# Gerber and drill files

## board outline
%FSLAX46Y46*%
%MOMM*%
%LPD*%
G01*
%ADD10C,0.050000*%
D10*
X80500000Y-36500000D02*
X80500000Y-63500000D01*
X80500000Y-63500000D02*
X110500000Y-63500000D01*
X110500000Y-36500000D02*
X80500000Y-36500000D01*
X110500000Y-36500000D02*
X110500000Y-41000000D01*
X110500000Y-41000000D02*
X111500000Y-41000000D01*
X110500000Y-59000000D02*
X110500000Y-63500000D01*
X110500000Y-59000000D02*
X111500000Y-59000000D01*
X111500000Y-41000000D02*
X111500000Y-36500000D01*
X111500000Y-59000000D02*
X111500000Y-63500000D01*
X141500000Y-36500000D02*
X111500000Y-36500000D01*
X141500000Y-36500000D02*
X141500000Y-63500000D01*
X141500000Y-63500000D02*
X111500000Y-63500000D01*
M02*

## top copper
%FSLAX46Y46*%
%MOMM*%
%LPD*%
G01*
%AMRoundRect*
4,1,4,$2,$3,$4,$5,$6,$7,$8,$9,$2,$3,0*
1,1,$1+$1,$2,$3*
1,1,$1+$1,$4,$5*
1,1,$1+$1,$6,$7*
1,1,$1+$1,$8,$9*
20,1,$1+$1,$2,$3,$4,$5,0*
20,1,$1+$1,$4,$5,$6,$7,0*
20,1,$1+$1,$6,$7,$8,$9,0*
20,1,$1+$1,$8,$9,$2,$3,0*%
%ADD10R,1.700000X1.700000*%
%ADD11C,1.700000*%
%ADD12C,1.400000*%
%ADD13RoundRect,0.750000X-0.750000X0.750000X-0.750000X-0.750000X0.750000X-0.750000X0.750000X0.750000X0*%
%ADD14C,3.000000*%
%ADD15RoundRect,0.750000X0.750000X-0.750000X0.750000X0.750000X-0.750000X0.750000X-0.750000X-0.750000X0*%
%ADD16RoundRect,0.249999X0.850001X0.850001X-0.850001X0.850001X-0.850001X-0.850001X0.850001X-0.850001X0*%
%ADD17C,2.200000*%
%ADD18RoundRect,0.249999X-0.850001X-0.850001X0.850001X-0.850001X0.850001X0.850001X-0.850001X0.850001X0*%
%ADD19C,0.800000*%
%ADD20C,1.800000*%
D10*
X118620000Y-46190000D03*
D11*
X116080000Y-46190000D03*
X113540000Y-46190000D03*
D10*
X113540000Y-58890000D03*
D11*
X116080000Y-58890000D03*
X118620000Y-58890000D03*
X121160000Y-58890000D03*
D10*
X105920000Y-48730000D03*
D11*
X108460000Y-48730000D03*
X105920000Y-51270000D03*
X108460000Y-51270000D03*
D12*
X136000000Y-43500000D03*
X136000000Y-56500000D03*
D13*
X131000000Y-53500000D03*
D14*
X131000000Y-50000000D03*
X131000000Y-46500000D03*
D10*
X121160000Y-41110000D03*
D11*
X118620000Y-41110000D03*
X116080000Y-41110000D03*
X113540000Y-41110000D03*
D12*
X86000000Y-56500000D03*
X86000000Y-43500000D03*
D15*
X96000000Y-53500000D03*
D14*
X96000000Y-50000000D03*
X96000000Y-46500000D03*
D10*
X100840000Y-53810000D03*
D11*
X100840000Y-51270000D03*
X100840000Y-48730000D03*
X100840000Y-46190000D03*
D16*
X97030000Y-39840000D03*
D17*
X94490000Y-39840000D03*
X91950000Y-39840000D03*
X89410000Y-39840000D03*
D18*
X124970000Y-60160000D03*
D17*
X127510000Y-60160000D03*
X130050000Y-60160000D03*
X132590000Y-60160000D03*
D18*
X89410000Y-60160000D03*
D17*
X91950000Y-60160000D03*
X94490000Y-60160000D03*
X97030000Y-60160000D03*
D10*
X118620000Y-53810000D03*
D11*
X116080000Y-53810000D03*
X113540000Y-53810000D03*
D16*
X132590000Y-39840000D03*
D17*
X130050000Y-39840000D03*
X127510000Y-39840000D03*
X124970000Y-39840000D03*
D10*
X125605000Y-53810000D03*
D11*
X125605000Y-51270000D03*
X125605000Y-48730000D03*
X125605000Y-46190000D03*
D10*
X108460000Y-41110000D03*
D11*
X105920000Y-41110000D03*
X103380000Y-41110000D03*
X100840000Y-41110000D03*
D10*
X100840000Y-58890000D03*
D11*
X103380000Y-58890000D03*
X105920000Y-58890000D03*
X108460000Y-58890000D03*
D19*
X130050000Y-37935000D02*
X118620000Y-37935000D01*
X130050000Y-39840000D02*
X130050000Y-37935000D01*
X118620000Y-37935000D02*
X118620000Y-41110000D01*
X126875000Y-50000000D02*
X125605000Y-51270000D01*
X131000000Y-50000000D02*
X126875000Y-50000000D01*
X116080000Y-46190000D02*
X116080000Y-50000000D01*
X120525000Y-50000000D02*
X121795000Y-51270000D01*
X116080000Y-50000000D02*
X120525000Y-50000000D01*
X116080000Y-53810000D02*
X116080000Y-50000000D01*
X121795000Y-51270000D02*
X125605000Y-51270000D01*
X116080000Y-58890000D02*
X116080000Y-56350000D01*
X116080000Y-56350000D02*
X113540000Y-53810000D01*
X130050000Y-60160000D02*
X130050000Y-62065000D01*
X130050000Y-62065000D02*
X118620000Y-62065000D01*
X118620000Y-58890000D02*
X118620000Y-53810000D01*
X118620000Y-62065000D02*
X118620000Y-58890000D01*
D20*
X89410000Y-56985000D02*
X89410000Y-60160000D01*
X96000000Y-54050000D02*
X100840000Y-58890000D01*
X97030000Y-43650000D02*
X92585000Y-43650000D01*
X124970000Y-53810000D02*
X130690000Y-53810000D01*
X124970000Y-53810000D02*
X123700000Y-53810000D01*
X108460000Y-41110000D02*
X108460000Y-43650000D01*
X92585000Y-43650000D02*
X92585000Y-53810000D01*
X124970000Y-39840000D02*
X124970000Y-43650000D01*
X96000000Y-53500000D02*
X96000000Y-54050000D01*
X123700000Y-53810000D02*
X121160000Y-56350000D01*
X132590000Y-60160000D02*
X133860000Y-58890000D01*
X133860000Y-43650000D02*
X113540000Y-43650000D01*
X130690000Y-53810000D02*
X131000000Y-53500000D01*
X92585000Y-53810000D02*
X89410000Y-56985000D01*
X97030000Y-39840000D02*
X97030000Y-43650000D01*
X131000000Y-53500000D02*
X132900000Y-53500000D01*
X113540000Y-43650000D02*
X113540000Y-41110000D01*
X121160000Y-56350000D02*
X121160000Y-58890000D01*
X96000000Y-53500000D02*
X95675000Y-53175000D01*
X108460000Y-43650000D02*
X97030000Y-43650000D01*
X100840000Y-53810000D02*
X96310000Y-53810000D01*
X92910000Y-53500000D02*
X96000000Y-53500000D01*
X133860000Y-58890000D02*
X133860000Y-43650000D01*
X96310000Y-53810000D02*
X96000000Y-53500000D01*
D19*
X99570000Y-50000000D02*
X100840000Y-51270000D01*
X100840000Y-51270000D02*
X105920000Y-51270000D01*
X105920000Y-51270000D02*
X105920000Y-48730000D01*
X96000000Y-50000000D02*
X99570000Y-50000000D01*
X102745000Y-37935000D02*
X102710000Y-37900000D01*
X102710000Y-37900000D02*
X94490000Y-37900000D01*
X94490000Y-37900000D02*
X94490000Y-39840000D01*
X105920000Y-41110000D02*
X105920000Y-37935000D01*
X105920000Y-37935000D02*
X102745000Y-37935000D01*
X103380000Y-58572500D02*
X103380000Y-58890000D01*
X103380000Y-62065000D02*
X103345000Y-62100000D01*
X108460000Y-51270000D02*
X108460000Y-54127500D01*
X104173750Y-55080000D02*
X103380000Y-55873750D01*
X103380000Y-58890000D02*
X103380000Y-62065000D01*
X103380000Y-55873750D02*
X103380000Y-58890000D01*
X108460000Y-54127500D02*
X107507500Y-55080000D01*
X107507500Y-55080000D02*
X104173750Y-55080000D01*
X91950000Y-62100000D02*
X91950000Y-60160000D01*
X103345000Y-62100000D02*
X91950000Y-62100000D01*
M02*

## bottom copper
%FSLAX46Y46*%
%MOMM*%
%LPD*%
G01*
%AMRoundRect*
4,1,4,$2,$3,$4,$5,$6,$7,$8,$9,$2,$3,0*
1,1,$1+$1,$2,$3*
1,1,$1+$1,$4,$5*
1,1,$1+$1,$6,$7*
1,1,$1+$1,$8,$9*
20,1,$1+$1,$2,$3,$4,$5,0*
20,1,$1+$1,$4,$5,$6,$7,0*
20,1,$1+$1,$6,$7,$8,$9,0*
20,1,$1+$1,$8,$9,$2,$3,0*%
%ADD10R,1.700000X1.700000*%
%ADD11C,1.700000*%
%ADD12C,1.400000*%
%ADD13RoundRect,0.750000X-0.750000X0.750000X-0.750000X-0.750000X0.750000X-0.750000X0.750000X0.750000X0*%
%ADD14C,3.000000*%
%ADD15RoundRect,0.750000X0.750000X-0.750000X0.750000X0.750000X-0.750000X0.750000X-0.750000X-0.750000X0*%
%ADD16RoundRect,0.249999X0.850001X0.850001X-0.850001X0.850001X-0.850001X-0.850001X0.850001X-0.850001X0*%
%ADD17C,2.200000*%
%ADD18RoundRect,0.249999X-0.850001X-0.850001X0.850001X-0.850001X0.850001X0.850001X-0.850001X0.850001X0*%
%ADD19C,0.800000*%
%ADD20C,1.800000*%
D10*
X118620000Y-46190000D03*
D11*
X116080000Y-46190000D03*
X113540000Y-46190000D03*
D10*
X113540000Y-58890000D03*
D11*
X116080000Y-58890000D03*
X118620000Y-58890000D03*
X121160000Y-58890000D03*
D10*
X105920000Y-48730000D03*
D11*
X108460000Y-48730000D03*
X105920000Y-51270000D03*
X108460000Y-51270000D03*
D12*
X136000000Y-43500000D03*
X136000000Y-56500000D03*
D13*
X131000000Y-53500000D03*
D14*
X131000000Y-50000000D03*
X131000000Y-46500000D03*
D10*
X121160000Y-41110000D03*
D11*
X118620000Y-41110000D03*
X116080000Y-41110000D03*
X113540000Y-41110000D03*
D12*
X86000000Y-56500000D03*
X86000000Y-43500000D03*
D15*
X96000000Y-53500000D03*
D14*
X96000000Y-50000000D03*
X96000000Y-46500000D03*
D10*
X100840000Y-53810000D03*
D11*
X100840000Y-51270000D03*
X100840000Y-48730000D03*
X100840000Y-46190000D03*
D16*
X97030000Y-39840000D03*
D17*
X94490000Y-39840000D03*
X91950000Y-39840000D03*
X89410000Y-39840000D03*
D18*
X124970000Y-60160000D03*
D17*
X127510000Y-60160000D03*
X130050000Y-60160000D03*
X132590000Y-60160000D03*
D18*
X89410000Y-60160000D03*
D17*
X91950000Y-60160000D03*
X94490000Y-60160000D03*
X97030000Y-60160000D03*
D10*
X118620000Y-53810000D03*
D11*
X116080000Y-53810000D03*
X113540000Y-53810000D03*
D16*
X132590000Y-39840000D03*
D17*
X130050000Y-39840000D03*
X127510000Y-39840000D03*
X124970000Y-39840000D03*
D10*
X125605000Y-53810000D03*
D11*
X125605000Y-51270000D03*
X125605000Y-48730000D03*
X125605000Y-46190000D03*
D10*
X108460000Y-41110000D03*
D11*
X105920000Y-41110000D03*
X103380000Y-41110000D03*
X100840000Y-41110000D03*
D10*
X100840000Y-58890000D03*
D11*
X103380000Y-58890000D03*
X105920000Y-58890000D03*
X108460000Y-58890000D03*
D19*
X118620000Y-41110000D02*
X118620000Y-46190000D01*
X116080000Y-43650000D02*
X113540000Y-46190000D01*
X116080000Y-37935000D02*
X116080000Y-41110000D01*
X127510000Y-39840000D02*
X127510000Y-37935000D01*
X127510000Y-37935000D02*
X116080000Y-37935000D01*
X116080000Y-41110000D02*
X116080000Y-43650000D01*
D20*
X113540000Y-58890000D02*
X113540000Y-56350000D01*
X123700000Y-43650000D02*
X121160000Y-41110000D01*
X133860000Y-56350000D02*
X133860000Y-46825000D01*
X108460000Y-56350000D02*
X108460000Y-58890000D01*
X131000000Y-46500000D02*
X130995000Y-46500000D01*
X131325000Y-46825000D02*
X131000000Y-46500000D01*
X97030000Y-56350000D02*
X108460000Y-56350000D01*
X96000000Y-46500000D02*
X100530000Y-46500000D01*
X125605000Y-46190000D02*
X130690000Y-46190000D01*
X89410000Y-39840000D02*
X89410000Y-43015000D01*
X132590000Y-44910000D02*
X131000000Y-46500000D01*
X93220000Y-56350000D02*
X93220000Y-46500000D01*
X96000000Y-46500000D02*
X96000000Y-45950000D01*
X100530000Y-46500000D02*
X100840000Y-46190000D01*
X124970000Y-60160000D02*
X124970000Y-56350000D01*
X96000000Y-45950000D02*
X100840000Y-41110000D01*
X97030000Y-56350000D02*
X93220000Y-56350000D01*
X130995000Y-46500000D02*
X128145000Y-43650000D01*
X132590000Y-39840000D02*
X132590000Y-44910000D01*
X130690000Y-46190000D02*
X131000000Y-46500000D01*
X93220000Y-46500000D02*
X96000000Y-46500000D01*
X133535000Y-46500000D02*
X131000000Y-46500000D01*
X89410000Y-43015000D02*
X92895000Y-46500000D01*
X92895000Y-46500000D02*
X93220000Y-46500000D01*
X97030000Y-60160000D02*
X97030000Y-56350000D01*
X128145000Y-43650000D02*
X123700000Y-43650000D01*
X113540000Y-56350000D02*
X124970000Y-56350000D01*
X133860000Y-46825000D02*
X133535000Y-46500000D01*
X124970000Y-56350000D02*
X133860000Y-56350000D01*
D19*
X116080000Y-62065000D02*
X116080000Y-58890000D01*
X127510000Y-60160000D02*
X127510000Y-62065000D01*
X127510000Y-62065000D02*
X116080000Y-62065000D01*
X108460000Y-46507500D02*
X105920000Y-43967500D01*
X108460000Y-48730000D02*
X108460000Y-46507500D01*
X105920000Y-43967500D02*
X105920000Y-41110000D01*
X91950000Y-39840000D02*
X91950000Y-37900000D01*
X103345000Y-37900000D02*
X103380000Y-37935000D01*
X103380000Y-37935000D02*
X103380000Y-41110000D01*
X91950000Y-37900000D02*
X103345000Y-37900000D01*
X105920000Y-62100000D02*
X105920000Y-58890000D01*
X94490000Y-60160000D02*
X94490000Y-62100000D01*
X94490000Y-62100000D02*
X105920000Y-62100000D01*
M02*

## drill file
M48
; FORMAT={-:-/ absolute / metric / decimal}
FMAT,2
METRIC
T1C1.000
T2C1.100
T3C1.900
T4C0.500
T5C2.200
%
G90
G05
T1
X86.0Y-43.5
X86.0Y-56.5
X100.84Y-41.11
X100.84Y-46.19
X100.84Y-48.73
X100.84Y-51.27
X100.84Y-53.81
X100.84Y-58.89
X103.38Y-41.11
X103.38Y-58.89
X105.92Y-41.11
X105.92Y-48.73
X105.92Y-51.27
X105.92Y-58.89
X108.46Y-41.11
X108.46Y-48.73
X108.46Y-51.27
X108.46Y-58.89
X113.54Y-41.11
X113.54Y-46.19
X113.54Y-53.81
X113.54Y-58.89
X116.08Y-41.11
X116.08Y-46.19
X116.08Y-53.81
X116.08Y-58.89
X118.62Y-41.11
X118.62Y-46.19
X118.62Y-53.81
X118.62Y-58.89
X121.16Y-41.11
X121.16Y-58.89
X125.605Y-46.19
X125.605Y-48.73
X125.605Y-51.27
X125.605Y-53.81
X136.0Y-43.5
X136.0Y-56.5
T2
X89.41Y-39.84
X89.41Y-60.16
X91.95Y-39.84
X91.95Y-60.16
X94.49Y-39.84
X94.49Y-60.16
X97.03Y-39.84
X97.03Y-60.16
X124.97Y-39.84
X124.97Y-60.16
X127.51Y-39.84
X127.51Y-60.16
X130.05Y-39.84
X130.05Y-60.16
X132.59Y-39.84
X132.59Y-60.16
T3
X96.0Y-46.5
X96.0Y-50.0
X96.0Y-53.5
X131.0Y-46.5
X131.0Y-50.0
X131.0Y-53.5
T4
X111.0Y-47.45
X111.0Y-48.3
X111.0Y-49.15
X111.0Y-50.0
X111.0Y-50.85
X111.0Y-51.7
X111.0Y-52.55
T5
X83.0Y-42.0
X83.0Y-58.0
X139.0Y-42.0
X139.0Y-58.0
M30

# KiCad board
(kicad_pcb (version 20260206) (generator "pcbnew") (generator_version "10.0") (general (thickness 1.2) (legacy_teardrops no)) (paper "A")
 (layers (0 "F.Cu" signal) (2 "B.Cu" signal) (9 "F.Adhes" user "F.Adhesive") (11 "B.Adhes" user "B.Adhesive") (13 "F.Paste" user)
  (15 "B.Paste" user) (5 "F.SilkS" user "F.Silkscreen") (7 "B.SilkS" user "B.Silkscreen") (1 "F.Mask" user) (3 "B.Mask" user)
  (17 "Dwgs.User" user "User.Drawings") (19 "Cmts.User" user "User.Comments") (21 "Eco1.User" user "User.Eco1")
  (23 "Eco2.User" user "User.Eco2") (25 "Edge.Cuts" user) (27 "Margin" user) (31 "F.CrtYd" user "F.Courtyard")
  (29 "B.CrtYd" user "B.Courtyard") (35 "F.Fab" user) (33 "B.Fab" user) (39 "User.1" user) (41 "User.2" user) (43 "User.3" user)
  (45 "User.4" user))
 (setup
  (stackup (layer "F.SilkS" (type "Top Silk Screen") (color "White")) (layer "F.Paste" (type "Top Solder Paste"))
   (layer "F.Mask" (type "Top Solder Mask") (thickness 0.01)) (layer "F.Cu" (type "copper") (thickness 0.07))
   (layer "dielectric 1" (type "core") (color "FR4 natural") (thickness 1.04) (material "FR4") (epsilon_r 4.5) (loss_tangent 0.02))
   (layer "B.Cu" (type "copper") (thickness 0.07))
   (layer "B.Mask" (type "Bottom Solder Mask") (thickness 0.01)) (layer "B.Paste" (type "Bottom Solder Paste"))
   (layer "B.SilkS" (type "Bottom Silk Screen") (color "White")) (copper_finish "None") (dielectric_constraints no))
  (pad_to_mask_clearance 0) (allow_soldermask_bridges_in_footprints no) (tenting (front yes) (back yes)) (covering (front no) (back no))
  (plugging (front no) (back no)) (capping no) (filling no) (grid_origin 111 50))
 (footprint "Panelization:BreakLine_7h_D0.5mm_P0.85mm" (layer "F.Cu") (at 111 50 90)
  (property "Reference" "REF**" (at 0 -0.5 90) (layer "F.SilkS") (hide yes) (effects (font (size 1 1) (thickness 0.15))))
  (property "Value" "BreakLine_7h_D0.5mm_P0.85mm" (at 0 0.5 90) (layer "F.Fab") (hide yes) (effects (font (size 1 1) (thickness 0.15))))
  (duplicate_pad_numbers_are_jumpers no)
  (pad "" np_thru_hole circle (at -2.55 0 90) (size 0.5 0.5) (drill 0.5) (layers "*.Cu" "*.Mask"))
  (pad "" np_thru_hole circle (at -1.7 0 90) (size 0.5 0.5) (drill 0.5) (layers "*.Cu" "*.Mask"))
  (pad "" np_thru_hole circle (at -0.85 0 90) (size 0.5 0.5) (drill 0.5) (layers "*.Cu" "*.Mask"))
  (pad "" np_thru_hole circle (at 0 0 90) (size 0.5 0.5) (drill 0.5) (layers "*.Cu" "*.Mask"))
  (pad "" np_thru_hole circle (at 0.85 0 90) (size 0.5 0.5) (drill 0.5) (layers "*.Cu" "*.Mask"))
  (pad "" np_thru_hole circle (at 1.7 0 90) (size 0.5 0.5) (drill 0.5) (layers "*.Cu" "*.Mask"))
  (pad "" np_thru_hole circle (at 2.55 0 90) (size 0.5 0.5) (drill 0.5) (layers "*.Cu" "*.Mask")))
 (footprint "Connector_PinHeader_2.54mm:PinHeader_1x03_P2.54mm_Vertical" (layer "F.Cu") (at 118.62 46.19 -90)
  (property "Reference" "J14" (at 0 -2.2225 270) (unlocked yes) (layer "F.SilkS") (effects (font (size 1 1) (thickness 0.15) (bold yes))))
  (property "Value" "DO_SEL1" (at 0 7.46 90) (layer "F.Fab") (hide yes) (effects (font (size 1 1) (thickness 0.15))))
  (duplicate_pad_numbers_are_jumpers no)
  (pad "1" thru_hole rect (at 0 0 270) (size 1.7 1.7) (drill 1) (layers "*.Cu" "*.Mask") (remove_unused_layers no) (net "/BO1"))
  (pad "2" thru_hole circle (at 0 2.54 270) (size 1.7 1.7) (drill 1) (layers "*.Cu" "*.Mask") (remove_unused_layers no) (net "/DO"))
  (pad "3" thru_hole circle (at 0 5.08 270) (size 1.7 1.7) (drill 1) (layers "*.Cu" "*.Mask") (remove_unused_layers no) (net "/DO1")))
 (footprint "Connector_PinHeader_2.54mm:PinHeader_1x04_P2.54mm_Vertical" (layer "F.Cu") (at 113.54 58.89 90)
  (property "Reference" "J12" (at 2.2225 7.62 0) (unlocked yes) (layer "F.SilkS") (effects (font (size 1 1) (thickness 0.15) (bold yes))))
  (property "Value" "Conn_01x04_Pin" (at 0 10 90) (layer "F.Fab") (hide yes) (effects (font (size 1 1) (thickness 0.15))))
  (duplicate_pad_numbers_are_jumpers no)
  (pad "1" thru_hole rect (at 0 0 90) (size 1.7 1.7) (drill 1) (layers "*.Cu" "*.Mask") (remove_unused_layers no) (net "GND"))
  (pad "2" thru_hole circle (at 0 2.54 90) (size 1.7 1.7) (drill 1) (layers "*.Cu" "*.Mask") (remove_unused_layers no) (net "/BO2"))
  (pad "3" thru_hole circle (at 0 5.08 90) (size 1.7 1.7) (drill 1) (layers "*.Cu" "*.Mask") (remove_unused_layers no) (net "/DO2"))
  (pad "4" thru_hole circle (at 0 7.62 90) (size 1.7 1.7) (drill 1) (layers "*.Cu" "*.Mask") (remove_unused_layers no) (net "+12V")))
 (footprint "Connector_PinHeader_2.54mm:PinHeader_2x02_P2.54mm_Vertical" (layer "F.Cu") (at 105.92 48.73)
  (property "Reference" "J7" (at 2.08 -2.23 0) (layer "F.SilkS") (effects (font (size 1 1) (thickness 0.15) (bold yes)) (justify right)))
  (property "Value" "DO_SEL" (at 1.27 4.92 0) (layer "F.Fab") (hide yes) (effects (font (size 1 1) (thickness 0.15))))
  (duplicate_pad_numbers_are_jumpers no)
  (pad "1" thru_hole rect (at 0 0) (size 1.7 1.7) (drill 1) (layers "*.Cu" "*.Mask") (remove_unused_layers no) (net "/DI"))
  (pad "2" thru_hole circle (at 2.54 0) (size 1.7 1.7) (drill 1) (layers "*.Cu" "*.Mask") (remove_unused_layers no) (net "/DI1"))
  (pad "3" thru_hole circle (at 0 2.54) (size 1.7 1.7) (drill 1) (layers "*.Cu" "*.Mask") (remove_unused_layers no) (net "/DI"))
  (pad "4" thru_hole circle (at 2.54 2.54) (size 1.7 1.7) (drill 1) (layers "*.Cu" "*.Mask") (remove_unused_layers no) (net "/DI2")))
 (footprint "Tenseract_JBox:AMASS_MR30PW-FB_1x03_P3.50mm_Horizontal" (layer "F.Cu") (at 131 53.5 -90)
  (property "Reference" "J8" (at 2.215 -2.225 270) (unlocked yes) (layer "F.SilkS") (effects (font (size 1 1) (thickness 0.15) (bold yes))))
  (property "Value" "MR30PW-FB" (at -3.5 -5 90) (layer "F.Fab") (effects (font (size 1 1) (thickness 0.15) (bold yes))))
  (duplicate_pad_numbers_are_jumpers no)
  (pad "" thru_hole circle (at -10 -5 270) (size 1.4 1.4) (drill 1) (layers "*.Cu" "*.Mask") (remove_unused_layers no))
  (pad "" thru_hole circle (at 3 -5) (size 1.4 1.4) (drill 1) (layers "*.Cu" "*.Mask") (remove_unused_layers no))
  (pad "1" thru_hole roundrect (at 0 0 270) (size 3 3) (drill 1.9) (layers "*.Cu" "*.Mask") (remove_unused_layers no)
   (roundrect_rratio 0.25) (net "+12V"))
  (pad "2" thru_hole circle (at -3.5 0 270) (size 3 3) (drill 1.9) (layers "*.Cu" "*.Mask") (remove_unused_layers no) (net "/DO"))
  (pad "3" thru_hole circle (at -7 0 270) (size 3 3) (drill 1.9) (layers "*.Cu" "*.Mask") (remove_unused_layers no) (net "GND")))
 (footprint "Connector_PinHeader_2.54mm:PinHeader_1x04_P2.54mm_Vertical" (layer "F.Cu") (at 121.16 41.11 -90)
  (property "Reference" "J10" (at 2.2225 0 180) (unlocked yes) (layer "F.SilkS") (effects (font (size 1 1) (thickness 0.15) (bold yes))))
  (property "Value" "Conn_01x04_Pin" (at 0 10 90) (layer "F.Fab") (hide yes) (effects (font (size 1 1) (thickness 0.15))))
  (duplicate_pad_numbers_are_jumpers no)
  (pad "1" thru_hole rect (at 0 0 270) (size 1.7 1.7) (drill 1) (layers "*.Cu" "*.Mask") (remove_unused_layers no) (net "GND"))
  (pad "2" thru_hole circle (at 0 2.54 270) (size 1.7 1.7) (drill 1) (layers "*.Cu" "*.Mask") (remove_unused_layers no) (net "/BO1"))
  (pad "3" thru_hole circle (at 0 5.08 270) (size 1.7 1.7) (drill 1) (layers "*.Cu" "*.Mask") (remove_unused_layers no) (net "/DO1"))
  (pad "4" thru_hole circle (at 0 7.62 270) (size 1.7 1.7) (drill 1) (layers "*.Cu" "*.Mask") (remove_unused_layers no) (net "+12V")))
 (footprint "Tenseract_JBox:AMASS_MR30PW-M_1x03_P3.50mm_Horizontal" (layer "F.Cu") (at 96 53.5 90)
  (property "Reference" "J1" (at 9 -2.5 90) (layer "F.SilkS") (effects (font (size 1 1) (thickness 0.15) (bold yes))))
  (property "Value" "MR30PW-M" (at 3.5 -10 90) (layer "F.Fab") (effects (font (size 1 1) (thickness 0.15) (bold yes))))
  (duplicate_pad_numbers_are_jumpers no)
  (pad "" thru_hole circle (at -3 -10 90) (size 1.4 1.4) (drill 1) (layers "*.Cu" "*.Mask") (remove_unused_layers no))
  (pad "" thru_hole circle (at 10 -10 90) (size 1.4 1.4) (drill 1) (layers "*.Cu" "*.Mask") (remove_unused_layers no))
  (pad "1" thru_hole roundrect (at 0 0 90) (size 3 3) (drill 1.9) (layers "*.Cu" "*.Mask") (remove_unused_layers no) (roundrect_rratio 0.25)
   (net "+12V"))
  (pad "2" thru_hole circle (at 3.5 0 90) (size 3 3) (drill 1.9) (layers "*.Cu" "*.Mask") (remove_unused_layers no) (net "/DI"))
  (pad "3" thru_hole circle (at 7 0 90) (size 3 3) (drill 1.9) (layers "*.Cu" "*.Mask") (remove_unused_layers no) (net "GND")))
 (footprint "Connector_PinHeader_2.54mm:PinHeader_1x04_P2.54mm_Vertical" (layer "F.Cu") (at 100.84 53.81 180)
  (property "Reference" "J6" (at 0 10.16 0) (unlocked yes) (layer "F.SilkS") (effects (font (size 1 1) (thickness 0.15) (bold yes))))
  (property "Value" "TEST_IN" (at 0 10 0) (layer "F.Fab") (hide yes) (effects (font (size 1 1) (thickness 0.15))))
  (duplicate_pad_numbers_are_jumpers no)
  (pad "1" thru_hole rect (at 0 0 180) (size 1.7 1.7) (drill 1) (layers "*.Cu" "*.Mask") (remove_unused_layers no) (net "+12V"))
  (pad "2" thru_hole circle (at 0 2.54 180) (size 1.7 1.7) (drill 1) (layers "*.Cu" "*.Mask") (remove_unused_layers no) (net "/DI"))
  (pad "3" thru_hole circle (at 0 5.08 180) (size 1.7 1.7) (drill 1) (layers "*.Cu" "*.Mask") (remove_unused_layers no)
   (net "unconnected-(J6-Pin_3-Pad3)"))
  (pad "4" thru_hole circle (at 0 7.62 180) (size 1.7 1.7) (drill 1) (layers "*.Cu" "*.Mask") (remove_unused_layers no) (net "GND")))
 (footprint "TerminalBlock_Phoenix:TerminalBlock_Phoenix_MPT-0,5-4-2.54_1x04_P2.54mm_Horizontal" (layer "F.Cu") (at 97.03 39.84 180)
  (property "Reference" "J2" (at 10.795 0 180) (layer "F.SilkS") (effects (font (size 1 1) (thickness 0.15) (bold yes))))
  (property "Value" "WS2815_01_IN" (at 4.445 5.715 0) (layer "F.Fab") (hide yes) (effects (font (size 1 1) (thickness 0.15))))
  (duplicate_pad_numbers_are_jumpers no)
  (pad "1" thru_hole roundrect (at 0 0 180) (size 2.2 2.2) (drill 1.1) (layers "*.Cu" "*.Mask") (remove_unused_layers no)
   (roundrect_rratio 0.113636) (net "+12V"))
  (pad "2" thru_hole circle (at 2.54 0 180) (size 2.2 2.2) (drill 1.1) (layers "*.Cu" "*.Mask") (remove_unused_layers no) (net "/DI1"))
  (pad "3" thru_hole circle (at 5.08 0 180) (size 2.2 2.2) (drill 1.1) (layers "*.Cu" "*.Mask") (remove_unused_layers no) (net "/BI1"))
  (pad "4" thru_hole circle (at 7.62 0 180) (size 2.2 2.2) (drill 1.1) (layers "*.Cu" "*.Mask") (remove_unused_layers no) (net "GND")))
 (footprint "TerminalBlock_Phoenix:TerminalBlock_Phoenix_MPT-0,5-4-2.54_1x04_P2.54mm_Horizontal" (layer "F.Cu") (at 124.97 60.16)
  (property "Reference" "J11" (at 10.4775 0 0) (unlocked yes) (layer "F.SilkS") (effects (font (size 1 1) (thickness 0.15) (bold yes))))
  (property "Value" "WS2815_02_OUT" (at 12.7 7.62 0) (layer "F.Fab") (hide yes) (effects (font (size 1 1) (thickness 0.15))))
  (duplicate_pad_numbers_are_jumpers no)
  (pad "1" thru_hole roundrect (at 0 0) (size 2.2 2.2) (drill 1.1) (layers "*.Cu" "*.Mask") (remove_unused_layers no)
   (roundrect_rratio 0.113636) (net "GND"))
  (pad "2" thru_hole circle (at 2.54 0) (size 2.2 2.2) (drill 1.1) (layers "*.Cu" "*.Mask") (remove_unused_layers no) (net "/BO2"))
  (pad "3" thru_hole circle (at 5.08 0) (size 2.2 2.2) (drill 1.1) (layers "*.Cu" "*.Mask") (remove_unused_layers no) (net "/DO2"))
  (pad "4" thru_hole circle (at 7.62 0) (size 2.2 2.2) (drill 1.1) (layers "*.Cu" "*.Mask") (remove_unused_layers no) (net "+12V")))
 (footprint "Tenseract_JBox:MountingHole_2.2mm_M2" (layer "F.Cu") (at 139 58)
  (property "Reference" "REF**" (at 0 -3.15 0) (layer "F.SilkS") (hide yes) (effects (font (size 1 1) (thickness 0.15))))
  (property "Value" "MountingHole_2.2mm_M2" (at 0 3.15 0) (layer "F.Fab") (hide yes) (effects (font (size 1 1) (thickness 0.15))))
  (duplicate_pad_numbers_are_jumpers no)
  (pad "" np_thru_hole circle (at 0 0) (size 2.2 2.2) (drill 2.2) (layers "*.Cu" "*.Mask")))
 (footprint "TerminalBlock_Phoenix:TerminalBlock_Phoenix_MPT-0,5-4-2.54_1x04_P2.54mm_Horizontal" (layer "F.Cu") (at 89.41 60.16)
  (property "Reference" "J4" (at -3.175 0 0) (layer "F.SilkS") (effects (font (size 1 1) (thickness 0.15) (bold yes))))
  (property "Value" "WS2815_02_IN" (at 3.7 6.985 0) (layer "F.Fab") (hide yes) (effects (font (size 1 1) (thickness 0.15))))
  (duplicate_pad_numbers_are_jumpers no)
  (pad "1" thru_hole roundrect (at 0 0) (size 2.2 2.2) (drill 1.1) (layers "*.Cu" "*.Mask") (remove_unused_layers no)
   (roundrect_rratio 0.113636) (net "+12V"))
  (pad "2" thru_hole circle (at 2.54 0) (size 2.2 2.2) (drill 1.1) (layers "*.Cu" "*.Mask") (remove_unused_layers no) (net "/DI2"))
  (pad "3" thru_hole circle (at 5.08 0) (size 2.2 2.2) (drill 1.1) (layers "*.Cu" "*.Mask") (remove_unused_layers no) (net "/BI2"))
  (pad "4" thru_hole circle (at 7.62 0) (size 2.2 2.2) (drill 1.1) (layers "*.Cu" "*.Mask") (remove_unused_layers no) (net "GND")))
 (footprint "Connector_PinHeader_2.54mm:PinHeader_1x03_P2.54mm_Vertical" (layer "F.Cu") (at 118.62 53.81 -90)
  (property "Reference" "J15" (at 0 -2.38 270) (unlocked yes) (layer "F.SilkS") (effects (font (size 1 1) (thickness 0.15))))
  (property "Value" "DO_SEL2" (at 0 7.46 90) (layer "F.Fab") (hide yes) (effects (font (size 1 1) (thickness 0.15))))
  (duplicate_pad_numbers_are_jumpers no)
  (pad "1" thru_hole rect (at 0 0 270) (size 1.7 1.7) (drill 1) (layers "*.Cu" "*.Mask") (remove_unused_layers no) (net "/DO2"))
  (pad "2" thru_hole circle (at 0 2.54 270) (size 1.7 1.7) (drill 1) (layers "*.Cu" "*.Mask") (remove_unused_layers no) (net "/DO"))
  (pad "3" thru_hole circle (at 0 5.08 270) (size 1.7 1.7) (drill 1) (layers "*.Cu" "*.Mask") (remove_unused_layers no) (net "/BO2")))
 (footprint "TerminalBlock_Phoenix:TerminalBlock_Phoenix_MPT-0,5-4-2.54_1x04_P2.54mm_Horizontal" (layer "F.Cu") (at 132.59 39.84 180)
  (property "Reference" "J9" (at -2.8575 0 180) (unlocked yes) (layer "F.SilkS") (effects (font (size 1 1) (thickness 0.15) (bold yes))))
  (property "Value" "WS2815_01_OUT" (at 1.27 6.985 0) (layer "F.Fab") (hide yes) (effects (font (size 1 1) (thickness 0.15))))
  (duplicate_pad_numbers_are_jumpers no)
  (pad "1" thru_hole roundrect (at 0 0 180) (size 2.2 2.2) (drill 1.1) (layers "*.Cu" "*.Mask") (remove_unused_layers no)
   (roundrect_rratio 0.113636) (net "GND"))
  (pad "2" thru_hole circle (at 2.54 0 180) (size 2.2 2.2) (drill 1.1) (layers "*.Cu" "*.Mask") (remove_unused_layers no) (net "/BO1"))
  (pad "3" thru_hole circle (at 5.08 0 180) (size 2.2 2.2) (drill 1.1) (layers "*.Cu" "*.Mask") (remove_unused_layers no) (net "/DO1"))
  (pad "4" thru_hole circle (at 7.62 0 180) (size 2.2 2.2) (drill 1.1) (layers "*.Cu" "*.Mask") (remove_unused_layers no) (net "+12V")))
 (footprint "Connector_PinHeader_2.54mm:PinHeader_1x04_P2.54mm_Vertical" (layer "F.Cu") (at 125.605 53.81 180)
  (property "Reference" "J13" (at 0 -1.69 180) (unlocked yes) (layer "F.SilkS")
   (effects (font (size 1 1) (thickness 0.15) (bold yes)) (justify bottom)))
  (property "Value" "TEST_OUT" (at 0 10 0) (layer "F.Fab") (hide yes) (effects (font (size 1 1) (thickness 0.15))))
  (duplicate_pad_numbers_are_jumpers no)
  (pad "1" thru_hole rect (at 0 0 180) (size 1.7 1.7) (drill 1) (layers "*.Cu" "*.Mask") (remove_unused_layers no) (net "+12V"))
  (pad "2" thru_hole circle (at 0 2.54 180) (size 1.7 1.7) (drill 1) (layers "*.Cu" "*.Mask") (remove_unused_layers no) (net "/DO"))
  (pad "3" thru_hole circle (at 0 5.08 180) (size 1.7 1.7) (drill 1) (layers "*.Cu" "*.Mask") (remove_unused_layers no)
   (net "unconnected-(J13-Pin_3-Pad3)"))
  (pad "4" thru_hole circle (at 0 7.62 180) (size 1.7 1.7) (drill 1) (layers "*.Cu" "*.Mask") (remove_unused_layers no) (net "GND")))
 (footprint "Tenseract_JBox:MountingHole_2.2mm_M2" (layer "F.Cu") (at 83 58)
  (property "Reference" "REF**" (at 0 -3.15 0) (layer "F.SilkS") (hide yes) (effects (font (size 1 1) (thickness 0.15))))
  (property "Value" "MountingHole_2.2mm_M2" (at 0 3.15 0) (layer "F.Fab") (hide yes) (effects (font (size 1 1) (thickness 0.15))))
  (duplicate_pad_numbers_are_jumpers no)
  (pad "" np_thru_hole circle (at 0 0) (size 2.2 2.2) (drill 2.2) (layers "*.Cu" "*.Mask")))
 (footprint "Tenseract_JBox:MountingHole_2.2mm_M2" (layer "F.Cu") (at 139 42)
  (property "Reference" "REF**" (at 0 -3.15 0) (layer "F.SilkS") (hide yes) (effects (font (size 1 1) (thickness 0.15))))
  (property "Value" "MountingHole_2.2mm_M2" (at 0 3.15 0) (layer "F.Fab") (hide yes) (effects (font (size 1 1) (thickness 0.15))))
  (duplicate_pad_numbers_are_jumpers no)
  (pad "" np_thru_hole circle (at 0 0) (size 2.2 2.2) (drill 2.2) (layers "*.Cu" "*.Mask")))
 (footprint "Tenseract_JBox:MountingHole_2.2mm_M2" (layer "F.Cu") (at 83 42)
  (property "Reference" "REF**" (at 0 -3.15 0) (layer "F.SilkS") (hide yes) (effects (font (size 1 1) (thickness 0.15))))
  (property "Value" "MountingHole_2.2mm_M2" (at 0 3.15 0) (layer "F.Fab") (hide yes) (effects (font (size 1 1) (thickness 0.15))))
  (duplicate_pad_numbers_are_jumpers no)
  (pad "" np_thru_hole circle (at 0 0) (size 2.2 2.2) (drill 2.2) (layers "*.Cu" "*.Mask")))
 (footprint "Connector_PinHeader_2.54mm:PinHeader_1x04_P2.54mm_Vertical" (layer "F.Cu") (at 108.46 41.11 -90)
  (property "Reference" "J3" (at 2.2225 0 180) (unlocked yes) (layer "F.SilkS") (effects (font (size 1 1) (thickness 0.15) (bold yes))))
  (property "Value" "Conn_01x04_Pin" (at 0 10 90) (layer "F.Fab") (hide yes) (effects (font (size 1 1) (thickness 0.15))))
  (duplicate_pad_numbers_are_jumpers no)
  (pad "1" thru_hole rect (at 0 0 270) (size 1.7 1.7) (drill 1) (layers "*.Cu" "*.Mask") (remove_unused_layers no) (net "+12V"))
  (pad "2" thru_hole circle (at 0 2.54 270) (size 1.7 1.7) (drill 1) (layers "*.Cu" "*.Mask") (remove_unused_layers no) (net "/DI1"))
  (pad "3" thru_hole circle (at 0 5.08 270) (size 1.7 1.7) (drill 1) (layers "*.Cu" "*.Mask") (remove_unused_layers no) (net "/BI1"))
  (pad "4" thru_hole circle (at 0 7.62 270) (size 1.7 1.7) (drill 1) (layers "*.Cu" "*.Mask") (remove_unused_layers no) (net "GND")))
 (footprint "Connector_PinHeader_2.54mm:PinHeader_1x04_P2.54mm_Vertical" (layer "F.Cu") (at 100.84 58.89 90)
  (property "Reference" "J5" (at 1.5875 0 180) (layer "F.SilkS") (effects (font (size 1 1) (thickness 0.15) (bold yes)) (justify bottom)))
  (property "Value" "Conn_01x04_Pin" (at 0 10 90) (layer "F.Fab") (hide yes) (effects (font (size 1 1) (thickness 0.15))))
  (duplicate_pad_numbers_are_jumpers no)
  (pad "1" thru_hole rect (at 0 0 90) (size 1.7 1.7) (drill 1) (layers "*.Cu" "*.Mask") (remove_unused_layers no) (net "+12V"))
  (pad "2" thru_hole circle (at 0 2.54 90) (size 1.7 1.7) (drill 1) (layers "*.Cu" "*.Mask") (remove_unused_layers no) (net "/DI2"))
  (pad "3" thru_hole circle (at 0 5.08 90) (size 1.7 1.7) (drill 1) (layers "*.Cu" "*.Mask") (remove_unused_layers no) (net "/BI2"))
  (pad "4" thru_hole circle (at 0 7.62 90) (size 1.7 1.7) (drill 1) (layers "*.Cu" "*.Mask") (remove_unused_layers no) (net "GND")))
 (gr_line (start 80.5 36.5) (end 80.5 63.5) (stroke (width 0.05) (type default)) (layer "Edge.Cuts"))
 (gr_line (start 80.5 63.5) (end 110.5 63.5) (stroke (width 0.05) (type default)) (layer "Edge.Cuts"))
 (gr_line (start 110.5 36.5) (end 80.5 36.5) (stroke (width 0.05) (type default)) (layer "Edge.Cuts"))
 (gr_line (start 110.5 36.5) (end 110.5 41) (stroke (width 0.05) (type default)) (layer "Edge.Cuts"))
 (gr_line (start 110.5 41) (end 111.5 41) (stroke (width 0.05) (type default)) (layer "Edge.Cuts"))
 (gr_line (start 110.5 59) (end 110.5 63.5) (stroke (width 0.05) (type default)) (layer "Edge.Cuts"))
 (gr_line (start 110.5 59) (end 111.5 59) (stroke (width 0.05) (type default)) (layer "Edge.Cuts"))
 (gr_line (start 111.5 41) (end 111.5 36.5) (stroke (width 0.05) (type default)) (layer "Edge.Cuts"))
 (gr_line (start 111.5 59) (end 111.5 63.5) (stroke (width 0.05) (type default)) (layer "Edge.Cuts"))
 (gr_line (start 141.5 36.5) (end 111.5 36.5) (stroke (width 0.05) (type default)) (layer "Edge.Cuts"))
 (gr_line (start 141.5 36.5) (end 141.5 63.5) (stroke (width 0.05) (type default)) (layer "Edge.Cuts"))
 (gr_line (start 141.5 63.5) (end 111.5 63.5) (stroke (width 0.05) (type default)) (layer "Edge.Cuts"))
 (segment (start 130.05 37.935) (end 118.62 37.935) (width 0.8) (layer "F.Cu") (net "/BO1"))
 (segment (start 130.05 39.84) (end 130.05 37.935) (width 0.8) (layer "F.Cu") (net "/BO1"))
 (segment (start 118.62 37.935) (end 118.62 41.11) (width 0.8) (layer "F.Cu") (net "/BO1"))
 (segment (start 118.62 41.11) (end 118.62 46.19) (width 0.8) (layer "B.Cu") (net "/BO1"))
 (segment (start 126.875 50) (end 125.605 51.27) (width 0.8) (layer "F.Cu") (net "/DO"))
 (segment (start 131 50) (end 126.875 50) (width 0.8) (layer "F.Cu") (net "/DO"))
 (segment (start 116.08 46.19) (end 116.08 50) (width 0.8) (layer "F.Cu") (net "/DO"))
 (segment (start 120.525 50) (end 121.795 51.27) (width 0.8) (layer "F.Cu") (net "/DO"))
 (segment (start 116.08 50) (end 120.525 50) (width 0.8) (layer "F.Cu") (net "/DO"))
 (segment (start 116.08 53.81) (end 116.08 50) (width 0.8) (layer "F.Cu") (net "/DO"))
 (segment (start 121.795 51.27) (end 125.605 51.27) (width 0.8) (layer "F.Cu") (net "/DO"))
 (segment (start 116.08 43.65) (end 113.54 46.19) (width 0.8) (layer "B.Cu") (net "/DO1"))
 (segment (start 116.08 37.935) (end 116.08 41.11) (width 0.8) (layer "B.Cu") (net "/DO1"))
 (segment (start 127.51 39.84) (end 127.51 37.935) (width 0.8) (layer "B.Cu") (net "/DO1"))
 (segment (start 127.51 37.935) (end 116.08 37.935) (width 0.8) (layer "B.Cu") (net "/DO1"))
 (segment (start 116.08 41.11) (end 116.08 43.65) (width 0.8) (layer "B.Cu") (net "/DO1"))
 (segment (start 113.54 58.89) (end 113.54 56.35) (width 1.8) (layer "B.Cu") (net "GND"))
 (segment (start 123.7 43.65) (end 121.16 41.11) (width 1.8) (layer "B.Cu") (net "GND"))
 (segment (start 133.86 56.35) (end 133.86 46.825) (width 1.8) (layer "B.Cu") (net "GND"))
 (segment (start 108.46 56.35) (end 108.46 58.89) (width 1.8) (layer "B.Cu") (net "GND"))
 (segment (start 131 46.5) (end 130.995 46.5) (width 1.8) (layer "B.Cu") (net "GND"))
 (segment (start 131.325 46.825) (end 131 46.5) (width 1.8) (layer "B.Cu") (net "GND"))
 (segment (start 97.03 56.35) (end 108.46 56.35) (width 1.8) (layer "B.Cu") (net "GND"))
 (segment (start 96 46.5) (end 100.53 46.5) (width 1.8) (layer "B.Cu") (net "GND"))
 (segment (start 125.605 46.19) (end 130.69 46.19) (width 1.8) (layer "B.Cu") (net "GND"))
 (segment (start 89.41 39.84) (end 89.41 43.015) (width 1.8) (layer "B.Cu") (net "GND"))
 (segment (start 132.59 44.91) (end 131 46.5) (width 1.8) (layer "B.Cu") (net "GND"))
 (segment (start 93.22 56.35) (end 93.22 46.5) (width 1.8) (layer "B.Cu") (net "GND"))
 (segment (start 96 46.5) (end 96 45.95) (width 1.8) (layer "B.Cu") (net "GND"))
 (segment (start 100.53 46.5) (end 100.84 46.19) (width 1.8) (layer "B.Cu") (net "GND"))
 (segment (start 124.97 60.16) (end 124.97 56.35) (width 1.8) (layer "B.Cu") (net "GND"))
 (segment (start 96 45.95) (end 100.84 41.11) (width 1.8) (layer "B.Cu") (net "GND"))
 (segment (start 97.03 56.35) (end 93.22 56.35) (width 1.8) (layer "B.Cu") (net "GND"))
 (segment (start 130.995 46.5) (end 128.145 43.65) (width 1.8) (layer "B.Cu") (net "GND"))
 (segment (start 132.59 39.84) (end 132.59 44.91) (width 1.8) (layer "B.Cu") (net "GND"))
 (segment (start 130.69 46.19) (end 131 46.5) (width 1.8) (layer "B.Cu") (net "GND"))
 (segment (start 93.22 46.5) (end 96 46.5) (width 1.8) (layer "B.Cu") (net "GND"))
 (segment (start 133.535 46.5) (end 131 46.5) (width 1.8) (layer "B.Cu") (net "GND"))
 (segment (start 89.41 43.015) (end 92.895 46.5) (width 1.8) (layer "B.Cu") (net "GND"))
 (segment (start 92.895 46.5) (end 93.22 46.5) (width 1.8) (layer "B.Cu") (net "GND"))
 (segment (start 97.03 60.16) (end 97.03 56.35) (width 1.8) (layer "B.Cu") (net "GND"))
 (segment (start 128.145 43.65) (end 123.7 43.65) (width 1.8) (layer "B.Cu") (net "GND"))
 (segment (start 113.54 56.35) (end 124.97 56.35) (width 1.8) (layer "B.Cu") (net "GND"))
 (segment (start 133.86 46.825) (end 133.535 46.5) (width 1.8) (layer "B.Cu") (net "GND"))
 (segment (start 124.97 56.35) (end 133.86 56.35) (width 1.8) (layer "B.Cu") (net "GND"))
 (segment (start 116.08 58.89) (end 116.08 56.35) (width 0.8) (layer "F.Cu") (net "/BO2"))
 (segment (start 116.08 56.35) (end 113.54 53.81) (width 0.8) (layer "F.Cu") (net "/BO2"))
 (segment (start 116.08 62.065) (end 116.08 58.89) (width 0.8) (layer "B.Cu") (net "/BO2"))
 (segment (start 127.51 60.16) (end 127.51 62.065) (width 0.8) (layer "B.Cu") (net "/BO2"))
 (segment (start 127.51 62.065) (end 116.08 62.065) (width 0.8) (layer "B.Cu") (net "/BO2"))
 (segment (start 130.05 60.16) (end 130.05 62.065) (width 0.8) (layer "F.Cu") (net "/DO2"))
 (segment (start 130.05 62.065) (end 118.62 62.065) (width 0.8) (layer "F.Cu") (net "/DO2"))
 (segment (start 118.62 58.89) (end 118.62 53.81) (width 0.8) (layer "F.Cu") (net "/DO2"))
 (segment (start 118.62 62.065) (end 118.62 58.89) (width 0.8) (layer "F.Cu") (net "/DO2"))
 (segment (start 89.41 56.985) (end 89.41 60.16) (width 1.8) (layer "F.Cu") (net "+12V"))
 (segment (start 96 54.05) (end 100.84 58.89) (width 1.8) (layer "F.Cu") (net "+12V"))
 (segment (start 97.03 43.65) (end 92.585 43.65) (width 1.8) (layer "F.Cu") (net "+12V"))
 (segment (start 124.97 53.81) (end 130.69 53.81) (width 1.8) (layer "F.Cu") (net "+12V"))
 (segment (start 124.97 53.81) (end 123.7 53.81) (width 1.8) (layer "F.Cu") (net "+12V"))
 (segment (start 108.46 41.11) (end 108.46 43.65) (width 1.8) (layer "F.Cu") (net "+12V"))
 (segment (start 92.585 43.65) (end 92.585 53.81) (width 1.8) (layer "F.Cu") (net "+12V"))
 (segment (start 124.97 39.84) (end 124.97 43.65) (width 1.8) (layer "F.Cu") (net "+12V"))
 (segment (start 96 53.5) (end 96 54.05) (width 1.8) (layer "F.Cu") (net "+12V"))
 (segment (start 123.7 53.81) (end 121.16 56.35) (width 1.8) (layer "F.Cu") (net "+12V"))
 (segment (start 132.59 60.16) (end 133.86 58.89) (width 1.8) (layer "F.Cu") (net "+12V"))
 (segment (start 133.86 43.65) (end 113.54 43.65) (width 1.8) (layer "F.Cu") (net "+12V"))
 (segment (start 130.69 53.81) (end 131 53.5) (width 1.8) (layer "F.Cu") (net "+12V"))
 (segment (start 92.585 53.81) (end 89.41 56.985) (width 1.8) (layer "F.Cu") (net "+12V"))
 (segment (start 97.03 39.84) (end 97.03 43.65) (width 1.8) (layer "F.Cu") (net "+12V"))
 (segment (start 131 53.5) (end 132.9 53.5) (width 1.8) (layer "F.Cu") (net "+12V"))
 (segment (start 113.54 43.65) (end 113.54 41.11) (width 1.8) (layer "F.Cu") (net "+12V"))
 (segment (start 121.16 56.35) (end 121.16 58.89) (width 1.8) (layer "F.Cu") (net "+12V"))
 (segment (start 96 53.5) (end 95.675 53.175) (width 1.8) (layer "F.Cu") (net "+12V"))
 (segment (start 108.46 43.65) (end 97.03 43.65) (width 1.8) (layer "F.Cu") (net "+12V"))
 (segment (start 100.84 53.81) (end 96.31 53.81) (width 1.8) (layer "F.Cu") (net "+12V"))
 (segment (start 92.91 53.5) (end 96 53.5) (width 1.8) (layer "F.Cu") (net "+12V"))
 (segment (start 133.86 58.89) (end 133.86 43.65) (width 1.8) (layer "F.Cu") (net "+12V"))
 (segment (start 96.31 53.81) (end 96 53.5) (width 1.8) (layer "F.Cu") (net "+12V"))
 (segment (start 99.57 50) (end 100.84 51.27) (width 0.8) (layer "F.Cu") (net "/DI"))
 (segment (start 100.84 51.27) (end 105.92 51.27) (width 0.8) (layer "F.Cu") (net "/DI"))
 (segment (start 105.92 51.27) (end 105.92 48.73) (width 0.8) (layer "F.Cu") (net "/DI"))
 (segment (start 96 50) (end 99.57 50) (width 0.8) (layer "F.Cu") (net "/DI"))
 (segment (start 102.745 37.935) (end 102.71 37.9) (width 0.8) (layer "F.Cu") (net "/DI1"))
 (segment (start 102.71 37.9) (end 94.49 37.9) (width 0.8) (layer "F.Cu") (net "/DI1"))
 (segment (start 94.49 37.9) (end 94.49 39.84) (width 0.8) (layer "F.Cu") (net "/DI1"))
 (segment (start 105.92 41.11) (end 105.92 37.935) (width 0.8) (layer "F.Cu") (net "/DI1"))
 (segment (start 105.92 37.935) (end 102.745 37.935) (width 0.8) (layer "F.Cu") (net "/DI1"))
 (segment (start 108.46 46.5075) (end 105.92 43.9675) (width 0.8) (layer "B.Cu") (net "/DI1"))
 (segment (start 108.46 48.73) (end 108.46 46.5075) (width 0.8) (layer "B.Cu") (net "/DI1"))
 (segment (start 105.92 43.9675) (end 105.92 41.11) (width 0.8) (layer "B.Cu") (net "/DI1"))
 (segment (start 103.38 58.5725) (end 103.38 58.89) (width 0.8) (layer "F.Cu") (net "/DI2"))
 (segment (start 103.38 62.065) (end 103.345 62.1) (width 0.8) (layer "F.Cu") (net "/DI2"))
 (segment (start 108.46 51.27) (end 108.46 54.1275) (width 0.8) (layer "F.Cu") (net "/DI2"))
 (segment (start 104.17375 55.08) (end 103.38 55.87375) (width 0.8) (layer "F.Cu") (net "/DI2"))
 (segment (start 103.38 58.89) (end 103.38 62.065) (width 0.8) (layer "F.Cu") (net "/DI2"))
 (segment (start 103.38 55.87375) (end 103.38 58.89) (width 0.8) (layer "F.Cu") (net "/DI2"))
 (segment (start 108.46 54.1275) (end 107.5075 55.08) (width 0.8) (layer "F.Cu") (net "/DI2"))
 (segment (start 107.5075 55.08) (end 104.17375 55.08) (width 0.8) (layer "F.Cu") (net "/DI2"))
 (segment (start 91.95 62.1) (end 91.95 60.16) (width 0.8) (layer "F.Cu") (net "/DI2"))
 (segment (start 103.345 62.1) (end 91.95 62.1) (width 0.8) (layer "F.Cu") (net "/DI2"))
 (segment (start 91.95 39.84) (end 91.95 37.9) (width 0.8) (layer "B.Cu") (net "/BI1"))
 (segment (start 103.345 37.9) (end 103.38 37.935) (width 0.8) (layer "B.Cu") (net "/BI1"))
 (segment (start 103.38 37.935) (end 103.38 41.11) (width 0.8) (layer "B.Cu") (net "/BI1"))
 (segment (start 91.95 37.9) (end 103.345 37.9) (width 0.8) (layer "B.Cu") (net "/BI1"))
 (segment (start 105.92 62.1) (end 105.92 58.89) (width 0.8) (layer "B.Cu") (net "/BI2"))
 (segment (start 94.49 60.16) (end 94.49 62.1) (width 0.8) (layer "B.Cu") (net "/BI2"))
 (segment (start 94.49 62.1) (end 105.92 62.1) (width 0.8) (layer "B.Cu") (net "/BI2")))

